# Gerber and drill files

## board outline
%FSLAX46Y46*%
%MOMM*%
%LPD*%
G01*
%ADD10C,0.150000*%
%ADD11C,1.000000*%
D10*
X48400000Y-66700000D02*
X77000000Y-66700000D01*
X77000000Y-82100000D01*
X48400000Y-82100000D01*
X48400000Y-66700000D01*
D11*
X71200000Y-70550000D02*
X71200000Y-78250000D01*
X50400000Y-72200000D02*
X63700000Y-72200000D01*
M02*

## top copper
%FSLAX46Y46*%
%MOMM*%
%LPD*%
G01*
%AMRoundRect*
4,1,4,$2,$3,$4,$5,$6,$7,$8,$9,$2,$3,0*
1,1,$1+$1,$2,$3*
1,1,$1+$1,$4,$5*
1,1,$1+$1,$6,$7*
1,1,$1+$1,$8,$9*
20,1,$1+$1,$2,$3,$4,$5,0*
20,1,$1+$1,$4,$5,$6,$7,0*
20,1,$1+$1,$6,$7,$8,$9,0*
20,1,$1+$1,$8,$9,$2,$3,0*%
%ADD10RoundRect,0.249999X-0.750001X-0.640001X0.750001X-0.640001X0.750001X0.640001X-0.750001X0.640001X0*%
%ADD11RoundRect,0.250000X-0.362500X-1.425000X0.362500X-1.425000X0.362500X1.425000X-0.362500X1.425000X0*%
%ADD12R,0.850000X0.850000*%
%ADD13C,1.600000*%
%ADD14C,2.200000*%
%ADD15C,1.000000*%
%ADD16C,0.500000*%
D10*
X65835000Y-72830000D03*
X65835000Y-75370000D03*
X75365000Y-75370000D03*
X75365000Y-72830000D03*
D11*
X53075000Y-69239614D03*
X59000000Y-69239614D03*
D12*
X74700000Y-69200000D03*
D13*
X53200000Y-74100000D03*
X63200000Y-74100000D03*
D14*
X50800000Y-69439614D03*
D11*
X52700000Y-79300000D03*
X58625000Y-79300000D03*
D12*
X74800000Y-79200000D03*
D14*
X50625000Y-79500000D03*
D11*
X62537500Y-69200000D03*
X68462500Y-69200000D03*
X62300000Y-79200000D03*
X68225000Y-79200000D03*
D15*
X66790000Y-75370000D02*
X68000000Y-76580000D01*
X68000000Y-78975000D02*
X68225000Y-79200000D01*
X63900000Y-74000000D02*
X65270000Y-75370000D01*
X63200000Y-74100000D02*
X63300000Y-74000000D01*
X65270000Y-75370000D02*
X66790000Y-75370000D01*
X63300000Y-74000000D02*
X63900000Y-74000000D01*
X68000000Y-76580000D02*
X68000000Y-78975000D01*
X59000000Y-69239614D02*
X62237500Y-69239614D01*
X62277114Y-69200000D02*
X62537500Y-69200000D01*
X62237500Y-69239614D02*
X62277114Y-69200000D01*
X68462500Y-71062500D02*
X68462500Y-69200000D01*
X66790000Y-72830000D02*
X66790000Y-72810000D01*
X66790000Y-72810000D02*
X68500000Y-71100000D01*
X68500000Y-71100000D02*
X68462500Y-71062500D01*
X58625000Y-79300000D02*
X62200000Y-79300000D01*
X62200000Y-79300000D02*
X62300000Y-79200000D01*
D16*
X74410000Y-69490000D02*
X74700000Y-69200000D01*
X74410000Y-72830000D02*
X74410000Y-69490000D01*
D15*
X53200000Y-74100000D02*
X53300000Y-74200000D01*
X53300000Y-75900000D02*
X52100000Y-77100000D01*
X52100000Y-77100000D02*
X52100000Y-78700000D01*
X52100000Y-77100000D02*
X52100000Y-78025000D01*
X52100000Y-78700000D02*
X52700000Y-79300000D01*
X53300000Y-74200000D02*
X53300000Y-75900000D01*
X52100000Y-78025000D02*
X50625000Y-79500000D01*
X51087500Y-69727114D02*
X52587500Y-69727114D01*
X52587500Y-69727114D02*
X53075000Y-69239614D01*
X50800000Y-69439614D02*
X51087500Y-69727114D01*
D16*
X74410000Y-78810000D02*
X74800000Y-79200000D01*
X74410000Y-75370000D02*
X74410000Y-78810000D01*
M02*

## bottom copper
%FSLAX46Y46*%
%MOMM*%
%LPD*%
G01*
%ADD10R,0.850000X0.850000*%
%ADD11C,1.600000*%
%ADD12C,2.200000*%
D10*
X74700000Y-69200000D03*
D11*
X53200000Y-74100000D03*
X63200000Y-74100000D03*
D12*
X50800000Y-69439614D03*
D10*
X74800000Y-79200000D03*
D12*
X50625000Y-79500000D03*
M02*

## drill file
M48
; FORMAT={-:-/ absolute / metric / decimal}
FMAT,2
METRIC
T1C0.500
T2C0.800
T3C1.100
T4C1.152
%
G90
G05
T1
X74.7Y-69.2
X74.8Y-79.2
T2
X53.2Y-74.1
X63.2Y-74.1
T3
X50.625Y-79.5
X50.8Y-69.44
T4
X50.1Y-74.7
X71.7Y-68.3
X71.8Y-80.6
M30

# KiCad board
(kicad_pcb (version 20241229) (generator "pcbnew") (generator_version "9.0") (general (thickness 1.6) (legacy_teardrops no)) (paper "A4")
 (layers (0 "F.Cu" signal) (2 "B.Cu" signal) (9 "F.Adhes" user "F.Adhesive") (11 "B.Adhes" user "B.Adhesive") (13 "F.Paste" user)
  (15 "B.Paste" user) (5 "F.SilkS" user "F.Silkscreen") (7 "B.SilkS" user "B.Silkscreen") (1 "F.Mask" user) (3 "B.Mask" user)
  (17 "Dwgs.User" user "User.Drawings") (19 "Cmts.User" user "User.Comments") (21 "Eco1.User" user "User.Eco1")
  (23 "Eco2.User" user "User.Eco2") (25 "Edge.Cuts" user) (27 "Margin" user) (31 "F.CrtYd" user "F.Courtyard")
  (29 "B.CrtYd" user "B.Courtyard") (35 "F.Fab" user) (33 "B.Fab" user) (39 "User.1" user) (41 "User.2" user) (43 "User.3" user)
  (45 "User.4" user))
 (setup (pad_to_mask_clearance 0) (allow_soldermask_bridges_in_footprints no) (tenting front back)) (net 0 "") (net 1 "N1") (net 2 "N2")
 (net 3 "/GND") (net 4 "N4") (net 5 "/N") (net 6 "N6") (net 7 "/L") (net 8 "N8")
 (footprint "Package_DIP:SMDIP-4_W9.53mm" (layer "F.Cu") (at 70.6 74.1)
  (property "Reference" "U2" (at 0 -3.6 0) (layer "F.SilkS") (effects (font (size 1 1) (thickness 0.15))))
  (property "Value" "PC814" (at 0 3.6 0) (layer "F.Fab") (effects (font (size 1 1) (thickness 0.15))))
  (pad "1" smd roundrect (at -4.765 -1.27) (size 2 1.78) (layers "F.Cu" "F.Mask" "F.Paste") (roundrect_rratio 0.140449) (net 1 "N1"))
  (pad "2" smd roundrect (at -4.765 1.27) (size 2 1.78) (layers "F.Cu" "F.Mask" "F.Paste") (roundrect_rratio 0.140449) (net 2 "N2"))
  (pad "3" smd roundrect (at 4.765 1.27) (size 2 1.78) (layers "F.Cu" "F.Mask" "F.Paste") (roundrect_rratio 0.140449) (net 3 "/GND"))
  (pad "4" smd roundrect (at 4.765 -1.27) (size 2 1.78) (layers "F.Cu" "F.Mask" "F.Paste") (roundrect_rratio 0.140449) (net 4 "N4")))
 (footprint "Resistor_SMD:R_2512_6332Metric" (layer "F.Cu") (at 56.0375 69.239614)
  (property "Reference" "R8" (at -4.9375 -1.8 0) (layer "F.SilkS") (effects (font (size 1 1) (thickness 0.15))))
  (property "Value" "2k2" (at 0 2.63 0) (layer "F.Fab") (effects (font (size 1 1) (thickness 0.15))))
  (pad "1" smd roundrect (at -2.9625 0) (size 1.225 3.35) (layers "F.Cu" "F.Mask" "F.Paste") (roundrect_rratio 0.204082) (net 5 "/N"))
  (pad "2" smd roundrect (at 2.9625 0) (size 1.225 3.35) (layers "F.Cu" "F.Mask" "F.Paste") (roundrect_rratio 0.204082) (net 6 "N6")))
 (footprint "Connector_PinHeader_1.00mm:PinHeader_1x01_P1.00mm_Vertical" (layer "F.Cu") (at 74.7 69.2)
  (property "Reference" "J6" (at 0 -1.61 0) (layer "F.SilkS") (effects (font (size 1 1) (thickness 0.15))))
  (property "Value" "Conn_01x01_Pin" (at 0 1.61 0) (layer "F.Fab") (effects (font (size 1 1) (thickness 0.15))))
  (pad "1" thru_hole rect (at 0 0) (size 0.85 0.85) (drill 0.5) (layers "*.Cu" "*.Mask") (remove_unused_layers no) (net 4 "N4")))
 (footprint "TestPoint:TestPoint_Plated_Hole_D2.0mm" (layer "F.Cu") (at 50.1 74.7)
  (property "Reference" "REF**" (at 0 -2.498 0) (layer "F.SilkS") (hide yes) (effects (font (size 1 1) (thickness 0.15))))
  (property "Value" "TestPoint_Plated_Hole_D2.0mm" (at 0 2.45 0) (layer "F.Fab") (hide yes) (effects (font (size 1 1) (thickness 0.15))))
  (pad "" np_thru_hole circle (at 0 0) (size 1.152 1.152) (drill 1.152) (layers "*.Cu" "*.Mask")))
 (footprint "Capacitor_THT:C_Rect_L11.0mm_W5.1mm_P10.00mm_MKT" (layer "F.Cu") (at 53.2 74.1)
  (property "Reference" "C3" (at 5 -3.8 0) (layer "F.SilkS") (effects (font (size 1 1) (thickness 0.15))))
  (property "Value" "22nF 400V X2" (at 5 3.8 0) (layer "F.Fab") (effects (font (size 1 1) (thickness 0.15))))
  (pad "1" thru_hole circle (at 0 0) (size 1.6 1.6) (drill 0.8) (layers "*.Cu" "*.Mask") (remove_unused_layers no) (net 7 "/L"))
  (pad "2" thru_hole circle (at 10 0) (size 1.6 1.6) (drill 0.8) (layers "*.Cu" "*.Mask") (remove_unused_layers no) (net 2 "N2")))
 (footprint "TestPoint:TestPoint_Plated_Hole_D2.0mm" (layer "F.Cu") (at 71.7 68.3)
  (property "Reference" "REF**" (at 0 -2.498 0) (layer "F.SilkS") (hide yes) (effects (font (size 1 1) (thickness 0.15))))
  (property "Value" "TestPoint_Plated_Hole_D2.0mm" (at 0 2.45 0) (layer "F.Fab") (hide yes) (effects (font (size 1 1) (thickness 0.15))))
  (pad "" np_thru_hole circle (at 0 0) (size 1.152 1.152) (drill 1.152) (layers "*.Cu" "*.Mask")))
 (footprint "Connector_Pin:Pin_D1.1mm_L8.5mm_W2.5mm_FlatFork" (layer "F.Cu") (at 50.8 69.439614)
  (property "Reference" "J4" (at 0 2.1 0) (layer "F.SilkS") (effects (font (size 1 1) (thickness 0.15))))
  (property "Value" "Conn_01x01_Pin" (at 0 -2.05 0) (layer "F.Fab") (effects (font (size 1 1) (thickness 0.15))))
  (pad "1" thru_hole circle (at 0 0) (size 2.2 2.2) (drill 1.1) (layers "*.Cu" "*.Mask") (remove_unused_layers no) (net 5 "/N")))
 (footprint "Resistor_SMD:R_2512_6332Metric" (layer "F.Cu") (at 55.6625 79.3)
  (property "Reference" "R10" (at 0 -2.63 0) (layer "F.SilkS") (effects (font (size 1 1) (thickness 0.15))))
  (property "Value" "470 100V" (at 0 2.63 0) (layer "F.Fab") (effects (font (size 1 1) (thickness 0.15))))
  (pad "1" smd roundrect (at -2.9625 0) (size 1.225 3.35) (layers "F.Cu" "F.Mask" "F.Paste") (roundrect_rratio 0.204082) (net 7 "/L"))
  (pad "2" smd roundrect (at 2.9625 0) (size 1.225 3.35) (layers "F.Cu" "F.Mask" "F.Paste") (roundrect_rratio 0.204082) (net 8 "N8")))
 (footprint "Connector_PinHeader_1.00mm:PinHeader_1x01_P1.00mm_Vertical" (layer "F.Cu") (at 74.8 79.2)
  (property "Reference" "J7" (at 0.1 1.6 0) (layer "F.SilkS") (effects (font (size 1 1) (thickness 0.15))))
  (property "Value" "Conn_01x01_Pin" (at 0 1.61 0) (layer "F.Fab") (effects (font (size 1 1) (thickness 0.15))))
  (pad "1" thru_hole rect (at 0 0) (size 0.85 0.85) (drill 0.5) (layers "*.Cu" "*.Mask") (remove_unused_layers no) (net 3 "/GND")))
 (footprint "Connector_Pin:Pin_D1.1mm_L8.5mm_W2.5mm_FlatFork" (layer "F.Cu") (at 50.625 79.5)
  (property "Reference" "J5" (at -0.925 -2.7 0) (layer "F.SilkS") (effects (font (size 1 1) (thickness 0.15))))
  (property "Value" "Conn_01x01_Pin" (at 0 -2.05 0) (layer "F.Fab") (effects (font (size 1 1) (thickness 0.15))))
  (pad "1" thru_hole circle (at 0 0) (size 2.2 2.2) (drill 1.1) (layers "*.Cu" "*.Mask") (remove_unused_layers no) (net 7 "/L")))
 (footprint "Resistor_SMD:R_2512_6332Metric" (layer "F.Cu") (at 65.5 69.2)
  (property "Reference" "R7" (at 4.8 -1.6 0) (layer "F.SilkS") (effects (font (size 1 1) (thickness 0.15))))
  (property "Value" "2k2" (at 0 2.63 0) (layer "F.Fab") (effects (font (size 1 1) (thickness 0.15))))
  (pad "1" smd roundrect (at -2.9625 0) (size 1.225 3.35) (layers "F.Cu" "F.Mask" "F.Paste") (roundrect_rratio 0.204082) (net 6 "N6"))
  (pad "2" smd roundrect (at 2.9625 0) (size 1.225 3.35) (layers "F.Cu" "F.Mask" "F.Paste") (roundrect_rratio 0.204082) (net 1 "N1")))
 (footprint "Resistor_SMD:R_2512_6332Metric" (layer "F.Cu") (at 65.2625 79.2)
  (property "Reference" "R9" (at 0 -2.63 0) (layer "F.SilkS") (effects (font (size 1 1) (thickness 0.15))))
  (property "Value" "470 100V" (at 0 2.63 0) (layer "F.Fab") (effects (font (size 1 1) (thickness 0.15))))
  (pad "1" smd roundrect (at -2.9625 0) (size 1.225 3.35) (layers "F.Cu" "F.Mask" "F.Paste") (roundrect_rratio 0.204082) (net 8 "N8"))
  (pad "2" smd roundrect (at 2.9625 0) (size 1.225 3.35) (layers "F.Cu" "F.Mask" "F.Paste") (roundrect_rratio 0.204082) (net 2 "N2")))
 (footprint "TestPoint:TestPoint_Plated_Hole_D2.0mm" (layer "F.Cu") (at 71.8 80.6)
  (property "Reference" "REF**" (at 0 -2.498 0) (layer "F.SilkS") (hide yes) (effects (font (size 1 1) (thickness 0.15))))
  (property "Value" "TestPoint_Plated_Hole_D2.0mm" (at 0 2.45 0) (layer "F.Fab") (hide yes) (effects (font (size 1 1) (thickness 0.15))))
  (pad "" np_thru_hole circle (at 0 0) (size 1.152 1.152) (drill 1.152) (layers "*.Cu" "*.Mask")))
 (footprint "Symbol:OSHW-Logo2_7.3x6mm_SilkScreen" (layer "B.Cu") (at 66.7 75.2 180)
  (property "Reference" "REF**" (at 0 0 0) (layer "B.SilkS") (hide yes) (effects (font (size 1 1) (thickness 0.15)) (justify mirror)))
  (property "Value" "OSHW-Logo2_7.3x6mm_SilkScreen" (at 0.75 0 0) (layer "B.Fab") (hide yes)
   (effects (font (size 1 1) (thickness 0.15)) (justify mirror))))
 (gr_rect (start 48.4 66.7) (end 77 82.1) (stroke (width 0.15) (type default)) (fill no) (layer "Edge.Cuts"))
 (gr_line (start 71.2 70.55) (end 71.2 78.25) (stroke (width 1) (type solid)) (layer "Edge.Cuts"))
 (gr_line (start 50.4 72.2) (end 63.7 72.2) (stroke (width 1) (type solid)) (layer "Edge.Cuts"))
 (segment (start 66.79 75.37) (end 68 76.58) (width 1) (layer "F.Cu") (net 2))
 (segment (start 68 78.975) (end 68.225 79.2) (width 1) (layer "F.Cu") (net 2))
 (segment (start 63.9 74) (end 65.27 75.37) (width 1) (layer "F.Cu") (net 2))
 (segment (start 63.2 74.1) (end 63.3 74) (width 1) (layer "F.Cu") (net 2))
 (segment (start 65.27 75.37) (end 66.79 75.37) (width 1) (layer "F.Cu") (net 2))
 (segment (start 63.3 74) (end 63.9 74) (width 1) (layer "F.Cu") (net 2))
 (segment (start 68 76.58) (end 68 78.975) (width 1) (layer "F.Cu") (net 2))
 (segment (start 59 69.239614) (end 62.2375 69.239614) (width 1) (layer "F.Cu") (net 6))
 (segment (start 62.277114 69.2) (end 62.5375 69.2) (width 1) (layer "F.Cu") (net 6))
 (segment (start 62.2375 69.239614) (end 62.277114 69.2) (width 1) (layer "F.Cu") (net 6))
 (segment (start 68.4625 71.0625) (end 68.4625 69.2) (width 1) (layer "F.Cu") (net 1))
 (segment (start 66.79 72.83) (end 66.79 72.81) (width 1) (layer "F.Cu") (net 1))
 (segment (start 66.79 72.81) (end 68.5 71.1) (width 1) (layer "F.Cu") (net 1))
 (segment (start 68.5 71.1) (end 68.4625 71.0625) (width 1) (layer "F.Cu") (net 1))
 (segment (start 58.625 79.3) (end 62.2 79.3) (width 1) (layer "F.Cu") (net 8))
 (segment (start 62.2 79.3) (end 62.3 79.2) (width 1) (layer "F.Cu") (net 8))
 (segment (start 74.41 69.49) (end 74.7 69.2) (width 0.5) (layer "F.Cu") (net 4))
 (segment (start 74.41 72.83) (end 74.41 69.49) (width 0.5) (layer "F.Cu") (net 4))
 (segment (start 53.2 74.1) (end 53.3 74.2) (width 1) (layer "F.Cu") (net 7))
 (segment (start 53.3 75.9) (end 52.1 77.1) (width 1) (layer "F.Cu") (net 7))
 (segment (start 52.1 77.1) (end 52.1 78.7) (width 1) (layer "F.Cu") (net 7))
 (segment (start 52.1 77.1) (end 52.1 78.025) (width 1) (layer "F.Cu") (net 7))
 (segment (start 52.1 78.7) (end 52.7 79.3) (width 1) (layer "F.Cu") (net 7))
 (segment (start 53.3 74.2) (end 53.3 75.9) (width 1) (layer "F.Cu") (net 7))
 (segment (start 52.1 78.025) (end 50.625 79.5) (width 1) (layer "F.Cu") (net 7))
 (segment (start 51.0875 69.727114) (end 52.5875 69.727114) (width 1) (layer "F.Cu") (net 5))
 (segment (start 52.5875 69.727114) (end 53.075 69.239614) (width 1) (layer "F.Cu") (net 5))
 (segment (start 50.8 69.439614) (end 51.0875 69.727114) (width 1) (layer "F.Cu") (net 5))
 (segment (start 74.41 78.81) (end 74.8 79.2) (width 0.5) (layer "F.Cu") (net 3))
 (segment (start 74.41 75.37) (end 74.41 78.81) (width 0.5) (layer "F.Cu") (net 3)))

